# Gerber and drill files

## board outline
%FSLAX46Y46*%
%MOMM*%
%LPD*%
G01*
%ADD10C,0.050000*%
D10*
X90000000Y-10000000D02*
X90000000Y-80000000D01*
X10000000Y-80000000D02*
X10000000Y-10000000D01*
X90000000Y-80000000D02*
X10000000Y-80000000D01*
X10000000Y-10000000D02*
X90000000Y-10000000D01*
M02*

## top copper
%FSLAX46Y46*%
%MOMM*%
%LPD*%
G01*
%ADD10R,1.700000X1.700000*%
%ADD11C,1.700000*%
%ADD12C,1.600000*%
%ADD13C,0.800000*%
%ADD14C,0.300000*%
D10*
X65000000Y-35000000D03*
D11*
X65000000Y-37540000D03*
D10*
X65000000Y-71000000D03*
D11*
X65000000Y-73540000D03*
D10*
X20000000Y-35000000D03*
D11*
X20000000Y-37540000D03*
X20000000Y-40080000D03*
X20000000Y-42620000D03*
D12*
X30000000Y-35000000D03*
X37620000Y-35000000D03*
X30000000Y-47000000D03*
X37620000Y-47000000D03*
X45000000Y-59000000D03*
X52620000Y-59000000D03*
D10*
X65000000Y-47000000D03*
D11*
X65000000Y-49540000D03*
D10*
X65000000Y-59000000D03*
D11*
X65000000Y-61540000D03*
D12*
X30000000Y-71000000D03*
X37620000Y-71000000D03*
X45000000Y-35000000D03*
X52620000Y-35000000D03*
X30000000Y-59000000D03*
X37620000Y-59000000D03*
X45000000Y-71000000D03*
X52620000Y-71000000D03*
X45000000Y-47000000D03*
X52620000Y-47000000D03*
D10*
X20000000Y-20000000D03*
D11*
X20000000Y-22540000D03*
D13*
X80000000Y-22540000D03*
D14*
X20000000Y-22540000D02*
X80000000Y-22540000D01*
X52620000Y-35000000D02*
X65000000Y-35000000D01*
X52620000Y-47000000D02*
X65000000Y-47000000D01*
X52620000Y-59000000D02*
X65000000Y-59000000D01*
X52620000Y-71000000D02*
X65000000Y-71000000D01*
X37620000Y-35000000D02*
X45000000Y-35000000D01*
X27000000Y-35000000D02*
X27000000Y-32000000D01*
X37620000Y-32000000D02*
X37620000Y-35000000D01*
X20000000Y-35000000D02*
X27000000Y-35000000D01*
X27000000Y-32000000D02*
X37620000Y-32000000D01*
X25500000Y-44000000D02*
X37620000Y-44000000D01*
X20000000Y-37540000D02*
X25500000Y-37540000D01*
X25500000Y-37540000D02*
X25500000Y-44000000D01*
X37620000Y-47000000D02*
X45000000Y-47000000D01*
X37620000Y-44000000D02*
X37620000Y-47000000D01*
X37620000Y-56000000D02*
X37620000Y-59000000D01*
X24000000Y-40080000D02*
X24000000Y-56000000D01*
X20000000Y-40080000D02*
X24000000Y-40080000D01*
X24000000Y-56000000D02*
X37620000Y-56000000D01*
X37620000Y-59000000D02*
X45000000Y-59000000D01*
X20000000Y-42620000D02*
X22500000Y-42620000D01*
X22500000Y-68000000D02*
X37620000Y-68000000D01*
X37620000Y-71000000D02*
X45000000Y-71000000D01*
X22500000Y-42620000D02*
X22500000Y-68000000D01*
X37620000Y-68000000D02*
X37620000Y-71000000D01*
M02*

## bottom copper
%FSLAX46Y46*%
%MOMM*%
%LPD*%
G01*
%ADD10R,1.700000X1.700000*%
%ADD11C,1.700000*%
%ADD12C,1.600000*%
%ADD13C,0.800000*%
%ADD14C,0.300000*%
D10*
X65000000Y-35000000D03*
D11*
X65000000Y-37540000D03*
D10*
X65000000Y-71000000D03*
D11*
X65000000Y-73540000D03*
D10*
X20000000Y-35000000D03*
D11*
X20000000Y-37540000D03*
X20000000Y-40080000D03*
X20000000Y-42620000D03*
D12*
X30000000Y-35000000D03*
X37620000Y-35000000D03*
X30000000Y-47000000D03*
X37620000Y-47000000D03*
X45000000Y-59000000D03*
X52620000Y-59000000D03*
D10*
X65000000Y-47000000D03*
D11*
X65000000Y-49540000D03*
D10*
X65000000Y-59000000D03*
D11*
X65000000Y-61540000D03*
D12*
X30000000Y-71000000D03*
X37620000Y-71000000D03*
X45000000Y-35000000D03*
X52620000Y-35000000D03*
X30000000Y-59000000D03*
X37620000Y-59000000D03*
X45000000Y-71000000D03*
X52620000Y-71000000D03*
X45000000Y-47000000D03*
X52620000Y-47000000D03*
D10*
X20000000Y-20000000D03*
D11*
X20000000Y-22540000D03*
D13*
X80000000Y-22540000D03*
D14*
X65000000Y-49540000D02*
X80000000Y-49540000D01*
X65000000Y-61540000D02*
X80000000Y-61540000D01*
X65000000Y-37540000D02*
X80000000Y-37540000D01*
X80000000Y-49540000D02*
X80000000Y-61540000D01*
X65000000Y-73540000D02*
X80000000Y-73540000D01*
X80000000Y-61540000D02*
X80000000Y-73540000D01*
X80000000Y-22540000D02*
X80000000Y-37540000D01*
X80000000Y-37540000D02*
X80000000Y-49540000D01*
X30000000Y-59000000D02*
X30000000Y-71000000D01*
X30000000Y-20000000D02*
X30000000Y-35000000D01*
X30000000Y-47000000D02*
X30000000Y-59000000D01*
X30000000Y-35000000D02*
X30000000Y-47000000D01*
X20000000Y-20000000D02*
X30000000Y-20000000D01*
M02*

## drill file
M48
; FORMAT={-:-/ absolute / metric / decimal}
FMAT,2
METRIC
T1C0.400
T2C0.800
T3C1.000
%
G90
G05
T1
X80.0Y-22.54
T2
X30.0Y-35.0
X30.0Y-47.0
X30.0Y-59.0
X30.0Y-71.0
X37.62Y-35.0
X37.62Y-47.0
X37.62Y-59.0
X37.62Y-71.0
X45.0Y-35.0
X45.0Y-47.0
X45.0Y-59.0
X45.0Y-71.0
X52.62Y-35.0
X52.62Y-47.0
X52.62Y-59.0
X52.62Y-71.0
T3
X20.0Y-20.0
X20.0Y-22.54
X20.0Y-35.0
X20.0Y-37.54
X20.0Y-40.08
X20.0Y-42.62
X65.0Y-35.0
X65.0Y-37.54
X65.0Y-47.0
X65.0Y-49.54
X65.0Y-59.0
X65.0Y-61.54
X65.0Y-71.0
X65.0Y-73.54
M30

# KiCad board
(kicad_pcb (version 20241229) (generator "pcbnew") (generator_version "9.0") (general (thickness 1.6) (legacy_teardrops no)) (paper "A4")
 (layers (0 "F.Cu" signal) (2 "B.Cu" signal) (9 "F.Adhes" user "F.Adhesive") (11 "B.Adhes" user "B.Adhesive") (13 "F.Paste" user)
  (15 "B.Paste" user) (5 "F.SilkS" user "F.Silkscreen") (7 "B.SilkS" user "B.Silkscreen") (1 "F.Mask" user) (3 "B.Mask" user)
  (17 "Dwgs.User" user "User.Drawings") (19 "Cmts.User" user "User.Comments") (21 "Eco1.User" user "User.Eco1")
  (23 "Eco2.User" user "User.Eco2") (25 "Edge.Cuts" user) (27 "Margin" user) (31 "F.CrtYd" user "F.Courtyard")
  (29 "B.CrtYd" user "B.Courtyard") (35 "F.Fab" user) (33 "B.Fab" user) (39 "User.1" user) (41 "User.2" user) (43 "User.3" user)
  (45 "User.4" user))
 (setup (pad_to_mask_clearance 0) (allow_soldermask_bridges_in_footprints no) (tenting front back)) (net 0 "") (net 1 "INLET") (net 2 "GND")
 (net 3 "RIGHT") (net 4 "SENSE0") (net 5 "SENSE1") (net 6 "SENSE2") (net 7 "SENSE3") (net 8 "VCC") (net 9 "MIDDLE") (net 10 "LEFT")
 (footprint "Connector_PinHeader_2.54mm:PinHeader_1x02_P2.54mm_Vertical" (layer "F.Cu") (at 65 35)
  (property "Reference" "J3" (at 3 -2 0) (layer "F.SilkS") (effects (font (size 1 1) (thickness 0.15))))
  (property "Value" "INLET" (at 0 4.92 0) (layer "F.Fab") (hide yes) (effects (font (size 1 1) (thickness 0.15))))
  (pad "1" thru_hole rect (at 0 0) (size 1.7 1.7) (drill 1) (layers "*.Cu" "*.Mask") (remove_unused_layers no) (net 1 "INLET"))
  (pad "2" thru_hole circle (at 0 2.54) (size 1.7 1.7) (drill 1) (layers "*.Cu" "*.Mask") (remove_unused_layers no) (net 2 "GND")))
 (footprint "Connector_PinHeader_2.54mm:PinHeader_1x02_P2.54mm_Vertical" (layer "F.Cu") (at 65 71)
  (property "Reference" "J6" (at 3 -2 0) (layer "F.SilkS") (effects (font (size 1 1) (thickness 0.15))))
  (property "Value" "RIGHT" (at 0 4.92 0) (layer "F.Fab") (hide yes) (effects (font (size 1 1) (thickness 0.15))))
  (pad "1" thru_hole rect (at 0 0) (size 1.7 1.7) (drill 1) (layers "*.Cu" "*.Mask") (remove_unused_layers no) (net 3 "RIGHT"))
  (pad "2" thru_hole circle (at 0 2.54) (size 1.7 1.7) (drill 1) (layers "*.Cu" "*.Mask") (remove_unused_layers no) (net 2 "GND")))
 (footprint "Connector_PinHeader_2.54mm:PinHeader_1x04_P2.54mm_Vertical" (layer "F.Cu") (at 20 35)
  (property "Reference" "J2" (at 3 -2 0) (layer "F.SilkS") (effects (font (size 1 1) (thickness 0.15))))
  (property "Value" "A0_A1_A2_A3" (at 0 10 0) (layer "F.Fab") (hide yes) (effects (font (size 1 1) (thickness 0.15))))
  (pad "1" thru_hole rect (at 0 0) (size 1.7 1.7) (drill 1) (layers "*.Cu" "*.Mask") (remove_unused_layers no) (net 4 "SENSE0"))
  (pad "2" thru_hole circle (at 0 2.54) (size 1.7 1.7) (drill 1) (layers "*.Cu" "*.Mask") (remove_unused_layers no) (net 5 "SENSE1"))
  (pad "3" thru_hole circle (at 0 5.08) (size 1.7 1.7) (drill 1) (layers "*.Cu" "*.Mask") (remove_unused_layers no) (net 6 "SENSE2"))
  (pad "4" thru_hole circle (at 0 7.62) (size 1.7 1.7) (drill 1) (layers "*.Cu" "*.Mask") (remove_unused_layers no) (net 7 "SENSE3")))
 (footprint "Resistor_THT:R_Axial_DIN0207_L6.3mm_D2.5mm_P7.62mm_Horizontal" (layer "F.Cu") (at 30 35)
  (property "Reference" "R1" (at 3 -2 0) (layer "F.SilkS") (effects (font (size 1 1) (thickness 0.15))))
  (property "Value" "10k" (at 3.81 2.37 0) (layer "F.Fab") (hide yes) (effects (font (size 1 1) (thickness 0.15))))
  (pad "1" thru_hole circle (at 0 0) (size 1.6 1.6) (drill 0.8) (layers "*.Cu" "*.Mask") (remove_unused_layers no) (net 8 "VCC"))
  (pad "2" thru_hole circle (at 7.62 0) (size 1.6 1.6) (drill 0.8) (layers "*.Cu" "*.Mask") (remove_unused_layers no) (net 4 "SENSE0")))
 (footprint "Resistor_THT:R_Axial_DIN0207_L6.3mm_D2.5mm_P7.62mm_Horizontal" (layer "F.Cu") (at 30 47)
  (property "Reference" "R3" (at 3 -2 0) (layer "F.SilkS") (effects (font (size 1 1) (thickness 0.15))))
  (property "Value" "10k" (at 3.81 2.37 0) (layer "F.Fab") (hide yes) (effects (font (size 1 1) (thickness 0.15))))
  (pad "1" thru_hole circle (at 0 0) (size 1.6 1.6) (drill 0.8) (layers "*.Cu" "*.Mask") (remove_unused_layers no) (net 8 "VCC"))
  (pad "2" thru_hole circle (at 7.62 0) (size 1.6 1.6) (drill 0.8) (layers "*.Cu" "*.Mask") (remove_unused_layers no) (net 5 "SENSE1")))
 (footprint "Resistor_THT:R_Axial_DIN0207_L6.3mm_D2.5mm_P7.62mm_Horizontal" (layer "F.Cu") (at 45 59)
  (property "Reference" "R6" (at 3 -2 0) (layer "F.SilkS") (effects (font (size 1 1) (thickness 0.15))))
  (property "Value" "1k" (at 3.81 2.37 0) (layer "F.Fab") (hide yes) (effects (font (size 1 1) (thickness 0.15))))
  (pad "1" thru_hole circle (at 0 0) (size 1.6 1.6) (drill 0.8) (layers "*.Cu" "*.Mask") (remove_unused_layers no) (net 6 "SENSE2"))
  (pad "2" thru_hole circle (at 7.62 0) (size 1.6 1.6) (drill 0.8) (layers "*.Cu" "*.Mask") (remove_unused_layers no) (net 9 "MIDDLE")))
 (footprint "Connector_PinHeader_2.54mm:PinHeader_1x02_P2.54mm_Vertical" (layer "F.Cu") (at 65 47)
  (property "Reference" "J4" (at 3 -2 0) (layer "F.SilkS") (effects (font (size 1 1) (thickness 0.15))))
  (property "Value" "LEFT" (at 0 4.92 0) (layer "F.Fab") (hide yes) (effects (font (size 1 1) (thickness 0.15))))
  (pad "1" thru_hole rect (at 0 0) (size 1.7 1.7) (drill 1) (layers "*.Cu" "*.Mask") (remove_unused_layers no) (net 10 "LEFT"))
  (pad "2" thru_hole circle (at 0 2.54) (size 1.7 1.7) (drill 1) (layers "*.Cu" "*.Mask") (remove_unused_layers no) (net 2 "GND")))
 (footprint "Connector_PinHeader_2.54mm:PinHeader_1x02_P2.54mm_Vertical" (layer "F.Cu") (at 65 59)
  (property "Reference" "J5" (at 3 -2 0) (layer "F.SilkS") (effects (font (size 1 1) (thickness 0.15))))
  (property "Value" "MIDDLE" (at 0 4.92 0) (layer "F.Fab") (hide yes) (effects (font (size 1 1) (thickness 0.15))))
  (pad "1" thru_hole rect (at 0 0) (size 1.7 1.7) (drill 1) (layers "*.Cu" "*.Mask") (remove_unused_layers no) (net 9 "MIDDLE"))
  (pad "2" thru_hole circle (at 0 2.54) (size 1.7 1.7) (drill 1) (layers "*.Cu" "*.Mask") (remove_unused_layers no) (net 2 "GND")))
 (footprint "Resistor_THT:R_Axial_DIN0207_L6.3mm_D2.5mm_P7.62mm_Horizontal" (layer "F.Cu") (at 30 71)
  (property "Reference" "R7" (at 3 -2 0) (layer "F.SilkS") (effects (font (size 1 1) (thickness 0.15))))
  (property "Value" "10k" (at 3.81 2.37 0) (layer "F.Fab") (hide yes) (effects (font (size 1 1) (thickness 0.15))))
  (pad "1" thru_hole circle (at 0 0) (size 1.6 1.6) (drill 0.8) (layers "*.Cu" "*.Mask") (remove_unused_layers no) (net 8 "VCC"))
  (pad "2" thru_hole circle (at 7.62 0) (size 1.6 1.6) (drill 0.8) (layers "*.Cu" "*.Mask") (remove_unused_layers no) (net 7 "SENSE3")))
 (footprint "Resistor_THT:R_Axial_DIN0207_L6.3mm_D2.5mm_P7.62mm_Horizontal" (layer "F.Cu") (at 45 35)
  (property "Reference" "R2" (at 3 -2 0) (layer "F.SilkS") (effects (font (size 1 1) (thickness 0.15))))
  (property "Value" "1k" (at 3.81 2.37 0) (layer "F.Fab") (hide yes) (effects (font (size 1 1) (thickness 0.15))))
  (pad "1" thru_hole circle (at 0 0) (size 1.6 1.6) (drill 0.8) (layers "*.Cu" "*.Mask") (remove_unused_layers no) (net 4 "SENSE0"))
  (pad "2" thru_hole circle (at 7.62 0) (size 1.6 1.6) (drill 0.8) (layers "*.Cu" "*.Mask") (remove_unused_layers no) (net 1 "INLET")))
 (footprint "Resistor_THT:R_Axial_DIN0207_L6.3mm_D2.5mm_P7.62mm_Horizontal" (layer "F.Cu") (at 30 59)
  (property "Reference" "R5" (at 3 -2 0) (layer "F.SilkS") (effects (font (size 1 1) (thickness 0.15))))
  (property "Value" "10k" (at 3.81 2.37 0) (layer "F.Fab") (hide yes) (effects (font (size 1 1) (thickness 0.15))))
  (pad "1" thru_hole circle (at 0 0) (size 1.6 1.6) (drill 0.8) (layers "*.Cu" "*.Mask") (remove_unused_layers no) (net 8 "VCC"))
  (pad "2" thru_hole circle (at 7.62 0) (size 1.6 1.6) (drill 0.8) (layers "*.Cu" "*.Mask") (remove_unused_layers no) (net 6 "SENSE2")))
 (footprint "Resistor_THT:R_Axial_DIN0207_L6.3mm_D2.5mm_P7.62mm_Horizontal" (layer "F.Cu") (at 45 71)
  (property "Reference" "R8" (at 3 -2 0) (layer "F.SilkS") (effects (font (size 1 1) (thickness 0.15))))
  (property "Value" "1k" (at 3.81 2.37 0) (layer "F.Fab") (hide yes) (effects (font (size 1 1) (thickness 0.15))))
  (pad "1" thru_hole circle (at 0 0) (size 1.6 1.6) (drill 0.8) (layers "*.Cu" "*.Mask") (remove_unused_layers no) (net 7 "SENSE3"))
  (pad "2" thru_hole circle (at 7.62 0) (size 1.6 1.6) (drill 0.8) (layers "*.Cu" "*.Mask") (remove_unused_layers no) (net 3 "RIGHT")))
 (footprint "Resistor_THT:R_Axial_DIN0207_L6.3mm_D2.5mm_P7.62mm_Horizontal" (layer "F.Cu") (at 45 47)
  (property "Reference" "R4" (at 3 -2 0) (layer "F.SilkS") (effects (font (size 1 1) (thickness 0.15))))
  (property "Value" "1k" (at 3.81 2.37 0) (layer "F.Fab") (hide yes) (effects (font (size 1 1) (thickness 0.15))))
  (pad "1" thru_hole circle (at 0 0) (size 1.6 1.6) (drill 0.8) (layers "*.Cu" "*.Mask") (remove_unused_layers no) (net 5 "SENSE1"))
  (pad "2" thru_hole circle (at 7.62 0) (size 1.6 1.6) (drill 0.8) (layers "*.Cu" "*.Mask") (remove_unused_layers no) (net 10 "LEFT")))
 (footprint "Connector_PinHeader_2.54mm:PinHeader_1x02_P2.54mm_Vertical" (layer "F.Cu") (at 20 20)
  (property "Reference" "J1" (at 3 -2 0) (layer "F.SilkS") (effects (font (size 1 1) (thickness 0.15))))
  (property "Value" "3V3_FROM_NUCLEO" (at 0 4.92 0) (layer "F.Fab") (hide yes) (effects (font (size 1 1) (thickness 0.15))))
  (pad "1" thru_hole rect (at 0 0) (size 1.7 1.7) (drill 1) (layers "*.Cu" "*.Mask") (remove_unused_layers no) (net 8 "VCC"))
  (pad "2" thru_hole circle (at 0 2.54) (size 1.7 1.7) (drill 1) (layers "*.Cu" "*.Mask") (remove_unused_layers no) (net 2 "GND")))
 (gr_line (start 90 10) (end 90 80) (stroke (width 0.05) (type default)) (layer "Edge.Cuts"))
 (gr_line (start 10 80) (end 10 10) (stroke (width 0.05) (type default)) (layer "Edge.Cuts"))
 (gr_line (start 90 80) (end 10 80) (stroke (width 0.05) (type default)) (layer "Edge.Cuts"))
 (gr_line (start 10 10) (end 90 10) (stroke (width 0.05) (type default)) (layer "Edge.Cuts"))
 (segment (start 20 22.54) (end 80 22.54) (width 0.3) (layer "F.Cu") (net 2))
 (via (at 80 22.54) (size 0.8) (drill 0.4) (layers "F.Cu" "B.Cu") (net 2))
 (segment (start 65 49.54) (end 80 49.54) (width 0.3) (layer "B.Cu") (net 2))
 (segment (start 65 61.54) (end 80 61.54) (width 0.3) (layer "B.Cu") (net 2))
 (segment (start 65 37.54) (end 80 37.54) (width 0.3) (layer "B.Cu") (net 2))
 (segment (start 80 49.54) (end 80 61.54) (width 0.3) (layer "B.Cu") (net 2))
 (segment (start 65 73.54) (end 80 73.54) (width 0.3) (layer "B.Cu") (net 2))
 (segment (start 80 61.54) (end 80 73.54) (width 0.3) (layer "B.Cu") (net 2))
 (segment (start 80 22.54) (end 80 37.54) (width 0.3) (layer "B.Cu") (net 2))
 (segment (start 80 37.54) (end 80 49.54) (width 0.3) (layer "B.Cu") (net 2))
 (segment (start 52.62 35) (end 65 35) (width 0.3) (layer "F.Cu") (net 1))
 (segment (start 52.62 47) (end 65 47) (width 0.3) (layer "F.Cu") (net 10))
 (segment (start 52.62 59) (end 65 59) (width 0.3) (layer "F.Cu") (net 9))
 (segment (start 52.62 71) (end 65 71) (width 0.3) (layer "F.Cu") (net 3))
 (segment (start 37.62 35) (end 45 35) (width 0.3) (layer "F.Cu") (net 4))
 (segment (start 27 35) (end 27 32) (width 0.3) (layer "F.Cu") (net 4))
 (segment (start 37.62 32) (end 37.62 35) (width 0.3) (layer "F.Cu") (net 4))
 (segment (start 20 35) (end 27 35) (width 0.3) (layer "F.Cu") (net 4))
 (segment (start 27 32) (end 37.62 32) (width 0.3) (layer "F.Cu") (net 4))
 (segment (start 25.5 44) (end 37.62 44) (width 0.3) (layer "F.Cu") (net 5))
 (segment (start 20 37.54) (end 25.5 37.54) (width 0.3) (layer "F.Cu") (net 5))
 (segment (start 25.5 37.54) (end 25.5 44) (width 0.3) (layer "F.Cu") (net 5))
 (segment (start 37.62 47) (end 45 47) (width 0.3) (layer "F.Cu") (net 5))
 (segment (start 37.62 44) (end 37.62 47) (width 0.3) (layer "F.Cu") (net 5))
 (segment (start 37.62 56) (end 37.62 59) (width 0.3) (layer "F.Cu") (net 6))
 (segment (start 24 40.08) (end 24 56) (width 0.3) (layer "F.Cu") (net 6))
 (segment (start 20 40.08) (end 24 40.08) (width 0.3) (layer "F.Cu") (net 6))
 (segment (start 24 56) (end 37.62 56) (width 0.3) (layer "F.Cu") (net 6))
 (segment (start 37.62 59) (end 45 59) (width 0.3) (layer "F.Cu") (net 6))
 (segment (start 20 42.62) (end 22.5 42.62) (width 0.3) (layer "F.Cu") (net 7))
 (segment (start 22.5 68) (end 37.62 68) (width 0.3) (layer "F.Cu") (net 7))
 (segment (start 37.62 71) (end 45 71) (width 0.3) (layer "F.Cu") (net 7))
 (segment (start 22.5 42.62) (end 22.5 68) (width 0.3) (layer "F.Cu") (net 7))
 (segment (start 37.62 68) (end 37.62 71) (width 0.3) (layer "F.Cu") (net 7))
 (segment (start 30 59) (end 30 71) (width 0.3) (layer "B.Cu") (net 8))
 (segment (start 30 20) (end 30 35) (width 0.3) (layer "B.Cu") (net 8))
 (segment (start 30 47) (end 30 59) (width 0.3) (layer "B.Cu") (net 8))
 (segment (start 30 35) (end 30 47) (width 0.3) (layer "B.Cu") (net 8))
 (segment (start 20 20) (end 30 20) (width 0.3) (layer "B.Cu") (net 8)))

